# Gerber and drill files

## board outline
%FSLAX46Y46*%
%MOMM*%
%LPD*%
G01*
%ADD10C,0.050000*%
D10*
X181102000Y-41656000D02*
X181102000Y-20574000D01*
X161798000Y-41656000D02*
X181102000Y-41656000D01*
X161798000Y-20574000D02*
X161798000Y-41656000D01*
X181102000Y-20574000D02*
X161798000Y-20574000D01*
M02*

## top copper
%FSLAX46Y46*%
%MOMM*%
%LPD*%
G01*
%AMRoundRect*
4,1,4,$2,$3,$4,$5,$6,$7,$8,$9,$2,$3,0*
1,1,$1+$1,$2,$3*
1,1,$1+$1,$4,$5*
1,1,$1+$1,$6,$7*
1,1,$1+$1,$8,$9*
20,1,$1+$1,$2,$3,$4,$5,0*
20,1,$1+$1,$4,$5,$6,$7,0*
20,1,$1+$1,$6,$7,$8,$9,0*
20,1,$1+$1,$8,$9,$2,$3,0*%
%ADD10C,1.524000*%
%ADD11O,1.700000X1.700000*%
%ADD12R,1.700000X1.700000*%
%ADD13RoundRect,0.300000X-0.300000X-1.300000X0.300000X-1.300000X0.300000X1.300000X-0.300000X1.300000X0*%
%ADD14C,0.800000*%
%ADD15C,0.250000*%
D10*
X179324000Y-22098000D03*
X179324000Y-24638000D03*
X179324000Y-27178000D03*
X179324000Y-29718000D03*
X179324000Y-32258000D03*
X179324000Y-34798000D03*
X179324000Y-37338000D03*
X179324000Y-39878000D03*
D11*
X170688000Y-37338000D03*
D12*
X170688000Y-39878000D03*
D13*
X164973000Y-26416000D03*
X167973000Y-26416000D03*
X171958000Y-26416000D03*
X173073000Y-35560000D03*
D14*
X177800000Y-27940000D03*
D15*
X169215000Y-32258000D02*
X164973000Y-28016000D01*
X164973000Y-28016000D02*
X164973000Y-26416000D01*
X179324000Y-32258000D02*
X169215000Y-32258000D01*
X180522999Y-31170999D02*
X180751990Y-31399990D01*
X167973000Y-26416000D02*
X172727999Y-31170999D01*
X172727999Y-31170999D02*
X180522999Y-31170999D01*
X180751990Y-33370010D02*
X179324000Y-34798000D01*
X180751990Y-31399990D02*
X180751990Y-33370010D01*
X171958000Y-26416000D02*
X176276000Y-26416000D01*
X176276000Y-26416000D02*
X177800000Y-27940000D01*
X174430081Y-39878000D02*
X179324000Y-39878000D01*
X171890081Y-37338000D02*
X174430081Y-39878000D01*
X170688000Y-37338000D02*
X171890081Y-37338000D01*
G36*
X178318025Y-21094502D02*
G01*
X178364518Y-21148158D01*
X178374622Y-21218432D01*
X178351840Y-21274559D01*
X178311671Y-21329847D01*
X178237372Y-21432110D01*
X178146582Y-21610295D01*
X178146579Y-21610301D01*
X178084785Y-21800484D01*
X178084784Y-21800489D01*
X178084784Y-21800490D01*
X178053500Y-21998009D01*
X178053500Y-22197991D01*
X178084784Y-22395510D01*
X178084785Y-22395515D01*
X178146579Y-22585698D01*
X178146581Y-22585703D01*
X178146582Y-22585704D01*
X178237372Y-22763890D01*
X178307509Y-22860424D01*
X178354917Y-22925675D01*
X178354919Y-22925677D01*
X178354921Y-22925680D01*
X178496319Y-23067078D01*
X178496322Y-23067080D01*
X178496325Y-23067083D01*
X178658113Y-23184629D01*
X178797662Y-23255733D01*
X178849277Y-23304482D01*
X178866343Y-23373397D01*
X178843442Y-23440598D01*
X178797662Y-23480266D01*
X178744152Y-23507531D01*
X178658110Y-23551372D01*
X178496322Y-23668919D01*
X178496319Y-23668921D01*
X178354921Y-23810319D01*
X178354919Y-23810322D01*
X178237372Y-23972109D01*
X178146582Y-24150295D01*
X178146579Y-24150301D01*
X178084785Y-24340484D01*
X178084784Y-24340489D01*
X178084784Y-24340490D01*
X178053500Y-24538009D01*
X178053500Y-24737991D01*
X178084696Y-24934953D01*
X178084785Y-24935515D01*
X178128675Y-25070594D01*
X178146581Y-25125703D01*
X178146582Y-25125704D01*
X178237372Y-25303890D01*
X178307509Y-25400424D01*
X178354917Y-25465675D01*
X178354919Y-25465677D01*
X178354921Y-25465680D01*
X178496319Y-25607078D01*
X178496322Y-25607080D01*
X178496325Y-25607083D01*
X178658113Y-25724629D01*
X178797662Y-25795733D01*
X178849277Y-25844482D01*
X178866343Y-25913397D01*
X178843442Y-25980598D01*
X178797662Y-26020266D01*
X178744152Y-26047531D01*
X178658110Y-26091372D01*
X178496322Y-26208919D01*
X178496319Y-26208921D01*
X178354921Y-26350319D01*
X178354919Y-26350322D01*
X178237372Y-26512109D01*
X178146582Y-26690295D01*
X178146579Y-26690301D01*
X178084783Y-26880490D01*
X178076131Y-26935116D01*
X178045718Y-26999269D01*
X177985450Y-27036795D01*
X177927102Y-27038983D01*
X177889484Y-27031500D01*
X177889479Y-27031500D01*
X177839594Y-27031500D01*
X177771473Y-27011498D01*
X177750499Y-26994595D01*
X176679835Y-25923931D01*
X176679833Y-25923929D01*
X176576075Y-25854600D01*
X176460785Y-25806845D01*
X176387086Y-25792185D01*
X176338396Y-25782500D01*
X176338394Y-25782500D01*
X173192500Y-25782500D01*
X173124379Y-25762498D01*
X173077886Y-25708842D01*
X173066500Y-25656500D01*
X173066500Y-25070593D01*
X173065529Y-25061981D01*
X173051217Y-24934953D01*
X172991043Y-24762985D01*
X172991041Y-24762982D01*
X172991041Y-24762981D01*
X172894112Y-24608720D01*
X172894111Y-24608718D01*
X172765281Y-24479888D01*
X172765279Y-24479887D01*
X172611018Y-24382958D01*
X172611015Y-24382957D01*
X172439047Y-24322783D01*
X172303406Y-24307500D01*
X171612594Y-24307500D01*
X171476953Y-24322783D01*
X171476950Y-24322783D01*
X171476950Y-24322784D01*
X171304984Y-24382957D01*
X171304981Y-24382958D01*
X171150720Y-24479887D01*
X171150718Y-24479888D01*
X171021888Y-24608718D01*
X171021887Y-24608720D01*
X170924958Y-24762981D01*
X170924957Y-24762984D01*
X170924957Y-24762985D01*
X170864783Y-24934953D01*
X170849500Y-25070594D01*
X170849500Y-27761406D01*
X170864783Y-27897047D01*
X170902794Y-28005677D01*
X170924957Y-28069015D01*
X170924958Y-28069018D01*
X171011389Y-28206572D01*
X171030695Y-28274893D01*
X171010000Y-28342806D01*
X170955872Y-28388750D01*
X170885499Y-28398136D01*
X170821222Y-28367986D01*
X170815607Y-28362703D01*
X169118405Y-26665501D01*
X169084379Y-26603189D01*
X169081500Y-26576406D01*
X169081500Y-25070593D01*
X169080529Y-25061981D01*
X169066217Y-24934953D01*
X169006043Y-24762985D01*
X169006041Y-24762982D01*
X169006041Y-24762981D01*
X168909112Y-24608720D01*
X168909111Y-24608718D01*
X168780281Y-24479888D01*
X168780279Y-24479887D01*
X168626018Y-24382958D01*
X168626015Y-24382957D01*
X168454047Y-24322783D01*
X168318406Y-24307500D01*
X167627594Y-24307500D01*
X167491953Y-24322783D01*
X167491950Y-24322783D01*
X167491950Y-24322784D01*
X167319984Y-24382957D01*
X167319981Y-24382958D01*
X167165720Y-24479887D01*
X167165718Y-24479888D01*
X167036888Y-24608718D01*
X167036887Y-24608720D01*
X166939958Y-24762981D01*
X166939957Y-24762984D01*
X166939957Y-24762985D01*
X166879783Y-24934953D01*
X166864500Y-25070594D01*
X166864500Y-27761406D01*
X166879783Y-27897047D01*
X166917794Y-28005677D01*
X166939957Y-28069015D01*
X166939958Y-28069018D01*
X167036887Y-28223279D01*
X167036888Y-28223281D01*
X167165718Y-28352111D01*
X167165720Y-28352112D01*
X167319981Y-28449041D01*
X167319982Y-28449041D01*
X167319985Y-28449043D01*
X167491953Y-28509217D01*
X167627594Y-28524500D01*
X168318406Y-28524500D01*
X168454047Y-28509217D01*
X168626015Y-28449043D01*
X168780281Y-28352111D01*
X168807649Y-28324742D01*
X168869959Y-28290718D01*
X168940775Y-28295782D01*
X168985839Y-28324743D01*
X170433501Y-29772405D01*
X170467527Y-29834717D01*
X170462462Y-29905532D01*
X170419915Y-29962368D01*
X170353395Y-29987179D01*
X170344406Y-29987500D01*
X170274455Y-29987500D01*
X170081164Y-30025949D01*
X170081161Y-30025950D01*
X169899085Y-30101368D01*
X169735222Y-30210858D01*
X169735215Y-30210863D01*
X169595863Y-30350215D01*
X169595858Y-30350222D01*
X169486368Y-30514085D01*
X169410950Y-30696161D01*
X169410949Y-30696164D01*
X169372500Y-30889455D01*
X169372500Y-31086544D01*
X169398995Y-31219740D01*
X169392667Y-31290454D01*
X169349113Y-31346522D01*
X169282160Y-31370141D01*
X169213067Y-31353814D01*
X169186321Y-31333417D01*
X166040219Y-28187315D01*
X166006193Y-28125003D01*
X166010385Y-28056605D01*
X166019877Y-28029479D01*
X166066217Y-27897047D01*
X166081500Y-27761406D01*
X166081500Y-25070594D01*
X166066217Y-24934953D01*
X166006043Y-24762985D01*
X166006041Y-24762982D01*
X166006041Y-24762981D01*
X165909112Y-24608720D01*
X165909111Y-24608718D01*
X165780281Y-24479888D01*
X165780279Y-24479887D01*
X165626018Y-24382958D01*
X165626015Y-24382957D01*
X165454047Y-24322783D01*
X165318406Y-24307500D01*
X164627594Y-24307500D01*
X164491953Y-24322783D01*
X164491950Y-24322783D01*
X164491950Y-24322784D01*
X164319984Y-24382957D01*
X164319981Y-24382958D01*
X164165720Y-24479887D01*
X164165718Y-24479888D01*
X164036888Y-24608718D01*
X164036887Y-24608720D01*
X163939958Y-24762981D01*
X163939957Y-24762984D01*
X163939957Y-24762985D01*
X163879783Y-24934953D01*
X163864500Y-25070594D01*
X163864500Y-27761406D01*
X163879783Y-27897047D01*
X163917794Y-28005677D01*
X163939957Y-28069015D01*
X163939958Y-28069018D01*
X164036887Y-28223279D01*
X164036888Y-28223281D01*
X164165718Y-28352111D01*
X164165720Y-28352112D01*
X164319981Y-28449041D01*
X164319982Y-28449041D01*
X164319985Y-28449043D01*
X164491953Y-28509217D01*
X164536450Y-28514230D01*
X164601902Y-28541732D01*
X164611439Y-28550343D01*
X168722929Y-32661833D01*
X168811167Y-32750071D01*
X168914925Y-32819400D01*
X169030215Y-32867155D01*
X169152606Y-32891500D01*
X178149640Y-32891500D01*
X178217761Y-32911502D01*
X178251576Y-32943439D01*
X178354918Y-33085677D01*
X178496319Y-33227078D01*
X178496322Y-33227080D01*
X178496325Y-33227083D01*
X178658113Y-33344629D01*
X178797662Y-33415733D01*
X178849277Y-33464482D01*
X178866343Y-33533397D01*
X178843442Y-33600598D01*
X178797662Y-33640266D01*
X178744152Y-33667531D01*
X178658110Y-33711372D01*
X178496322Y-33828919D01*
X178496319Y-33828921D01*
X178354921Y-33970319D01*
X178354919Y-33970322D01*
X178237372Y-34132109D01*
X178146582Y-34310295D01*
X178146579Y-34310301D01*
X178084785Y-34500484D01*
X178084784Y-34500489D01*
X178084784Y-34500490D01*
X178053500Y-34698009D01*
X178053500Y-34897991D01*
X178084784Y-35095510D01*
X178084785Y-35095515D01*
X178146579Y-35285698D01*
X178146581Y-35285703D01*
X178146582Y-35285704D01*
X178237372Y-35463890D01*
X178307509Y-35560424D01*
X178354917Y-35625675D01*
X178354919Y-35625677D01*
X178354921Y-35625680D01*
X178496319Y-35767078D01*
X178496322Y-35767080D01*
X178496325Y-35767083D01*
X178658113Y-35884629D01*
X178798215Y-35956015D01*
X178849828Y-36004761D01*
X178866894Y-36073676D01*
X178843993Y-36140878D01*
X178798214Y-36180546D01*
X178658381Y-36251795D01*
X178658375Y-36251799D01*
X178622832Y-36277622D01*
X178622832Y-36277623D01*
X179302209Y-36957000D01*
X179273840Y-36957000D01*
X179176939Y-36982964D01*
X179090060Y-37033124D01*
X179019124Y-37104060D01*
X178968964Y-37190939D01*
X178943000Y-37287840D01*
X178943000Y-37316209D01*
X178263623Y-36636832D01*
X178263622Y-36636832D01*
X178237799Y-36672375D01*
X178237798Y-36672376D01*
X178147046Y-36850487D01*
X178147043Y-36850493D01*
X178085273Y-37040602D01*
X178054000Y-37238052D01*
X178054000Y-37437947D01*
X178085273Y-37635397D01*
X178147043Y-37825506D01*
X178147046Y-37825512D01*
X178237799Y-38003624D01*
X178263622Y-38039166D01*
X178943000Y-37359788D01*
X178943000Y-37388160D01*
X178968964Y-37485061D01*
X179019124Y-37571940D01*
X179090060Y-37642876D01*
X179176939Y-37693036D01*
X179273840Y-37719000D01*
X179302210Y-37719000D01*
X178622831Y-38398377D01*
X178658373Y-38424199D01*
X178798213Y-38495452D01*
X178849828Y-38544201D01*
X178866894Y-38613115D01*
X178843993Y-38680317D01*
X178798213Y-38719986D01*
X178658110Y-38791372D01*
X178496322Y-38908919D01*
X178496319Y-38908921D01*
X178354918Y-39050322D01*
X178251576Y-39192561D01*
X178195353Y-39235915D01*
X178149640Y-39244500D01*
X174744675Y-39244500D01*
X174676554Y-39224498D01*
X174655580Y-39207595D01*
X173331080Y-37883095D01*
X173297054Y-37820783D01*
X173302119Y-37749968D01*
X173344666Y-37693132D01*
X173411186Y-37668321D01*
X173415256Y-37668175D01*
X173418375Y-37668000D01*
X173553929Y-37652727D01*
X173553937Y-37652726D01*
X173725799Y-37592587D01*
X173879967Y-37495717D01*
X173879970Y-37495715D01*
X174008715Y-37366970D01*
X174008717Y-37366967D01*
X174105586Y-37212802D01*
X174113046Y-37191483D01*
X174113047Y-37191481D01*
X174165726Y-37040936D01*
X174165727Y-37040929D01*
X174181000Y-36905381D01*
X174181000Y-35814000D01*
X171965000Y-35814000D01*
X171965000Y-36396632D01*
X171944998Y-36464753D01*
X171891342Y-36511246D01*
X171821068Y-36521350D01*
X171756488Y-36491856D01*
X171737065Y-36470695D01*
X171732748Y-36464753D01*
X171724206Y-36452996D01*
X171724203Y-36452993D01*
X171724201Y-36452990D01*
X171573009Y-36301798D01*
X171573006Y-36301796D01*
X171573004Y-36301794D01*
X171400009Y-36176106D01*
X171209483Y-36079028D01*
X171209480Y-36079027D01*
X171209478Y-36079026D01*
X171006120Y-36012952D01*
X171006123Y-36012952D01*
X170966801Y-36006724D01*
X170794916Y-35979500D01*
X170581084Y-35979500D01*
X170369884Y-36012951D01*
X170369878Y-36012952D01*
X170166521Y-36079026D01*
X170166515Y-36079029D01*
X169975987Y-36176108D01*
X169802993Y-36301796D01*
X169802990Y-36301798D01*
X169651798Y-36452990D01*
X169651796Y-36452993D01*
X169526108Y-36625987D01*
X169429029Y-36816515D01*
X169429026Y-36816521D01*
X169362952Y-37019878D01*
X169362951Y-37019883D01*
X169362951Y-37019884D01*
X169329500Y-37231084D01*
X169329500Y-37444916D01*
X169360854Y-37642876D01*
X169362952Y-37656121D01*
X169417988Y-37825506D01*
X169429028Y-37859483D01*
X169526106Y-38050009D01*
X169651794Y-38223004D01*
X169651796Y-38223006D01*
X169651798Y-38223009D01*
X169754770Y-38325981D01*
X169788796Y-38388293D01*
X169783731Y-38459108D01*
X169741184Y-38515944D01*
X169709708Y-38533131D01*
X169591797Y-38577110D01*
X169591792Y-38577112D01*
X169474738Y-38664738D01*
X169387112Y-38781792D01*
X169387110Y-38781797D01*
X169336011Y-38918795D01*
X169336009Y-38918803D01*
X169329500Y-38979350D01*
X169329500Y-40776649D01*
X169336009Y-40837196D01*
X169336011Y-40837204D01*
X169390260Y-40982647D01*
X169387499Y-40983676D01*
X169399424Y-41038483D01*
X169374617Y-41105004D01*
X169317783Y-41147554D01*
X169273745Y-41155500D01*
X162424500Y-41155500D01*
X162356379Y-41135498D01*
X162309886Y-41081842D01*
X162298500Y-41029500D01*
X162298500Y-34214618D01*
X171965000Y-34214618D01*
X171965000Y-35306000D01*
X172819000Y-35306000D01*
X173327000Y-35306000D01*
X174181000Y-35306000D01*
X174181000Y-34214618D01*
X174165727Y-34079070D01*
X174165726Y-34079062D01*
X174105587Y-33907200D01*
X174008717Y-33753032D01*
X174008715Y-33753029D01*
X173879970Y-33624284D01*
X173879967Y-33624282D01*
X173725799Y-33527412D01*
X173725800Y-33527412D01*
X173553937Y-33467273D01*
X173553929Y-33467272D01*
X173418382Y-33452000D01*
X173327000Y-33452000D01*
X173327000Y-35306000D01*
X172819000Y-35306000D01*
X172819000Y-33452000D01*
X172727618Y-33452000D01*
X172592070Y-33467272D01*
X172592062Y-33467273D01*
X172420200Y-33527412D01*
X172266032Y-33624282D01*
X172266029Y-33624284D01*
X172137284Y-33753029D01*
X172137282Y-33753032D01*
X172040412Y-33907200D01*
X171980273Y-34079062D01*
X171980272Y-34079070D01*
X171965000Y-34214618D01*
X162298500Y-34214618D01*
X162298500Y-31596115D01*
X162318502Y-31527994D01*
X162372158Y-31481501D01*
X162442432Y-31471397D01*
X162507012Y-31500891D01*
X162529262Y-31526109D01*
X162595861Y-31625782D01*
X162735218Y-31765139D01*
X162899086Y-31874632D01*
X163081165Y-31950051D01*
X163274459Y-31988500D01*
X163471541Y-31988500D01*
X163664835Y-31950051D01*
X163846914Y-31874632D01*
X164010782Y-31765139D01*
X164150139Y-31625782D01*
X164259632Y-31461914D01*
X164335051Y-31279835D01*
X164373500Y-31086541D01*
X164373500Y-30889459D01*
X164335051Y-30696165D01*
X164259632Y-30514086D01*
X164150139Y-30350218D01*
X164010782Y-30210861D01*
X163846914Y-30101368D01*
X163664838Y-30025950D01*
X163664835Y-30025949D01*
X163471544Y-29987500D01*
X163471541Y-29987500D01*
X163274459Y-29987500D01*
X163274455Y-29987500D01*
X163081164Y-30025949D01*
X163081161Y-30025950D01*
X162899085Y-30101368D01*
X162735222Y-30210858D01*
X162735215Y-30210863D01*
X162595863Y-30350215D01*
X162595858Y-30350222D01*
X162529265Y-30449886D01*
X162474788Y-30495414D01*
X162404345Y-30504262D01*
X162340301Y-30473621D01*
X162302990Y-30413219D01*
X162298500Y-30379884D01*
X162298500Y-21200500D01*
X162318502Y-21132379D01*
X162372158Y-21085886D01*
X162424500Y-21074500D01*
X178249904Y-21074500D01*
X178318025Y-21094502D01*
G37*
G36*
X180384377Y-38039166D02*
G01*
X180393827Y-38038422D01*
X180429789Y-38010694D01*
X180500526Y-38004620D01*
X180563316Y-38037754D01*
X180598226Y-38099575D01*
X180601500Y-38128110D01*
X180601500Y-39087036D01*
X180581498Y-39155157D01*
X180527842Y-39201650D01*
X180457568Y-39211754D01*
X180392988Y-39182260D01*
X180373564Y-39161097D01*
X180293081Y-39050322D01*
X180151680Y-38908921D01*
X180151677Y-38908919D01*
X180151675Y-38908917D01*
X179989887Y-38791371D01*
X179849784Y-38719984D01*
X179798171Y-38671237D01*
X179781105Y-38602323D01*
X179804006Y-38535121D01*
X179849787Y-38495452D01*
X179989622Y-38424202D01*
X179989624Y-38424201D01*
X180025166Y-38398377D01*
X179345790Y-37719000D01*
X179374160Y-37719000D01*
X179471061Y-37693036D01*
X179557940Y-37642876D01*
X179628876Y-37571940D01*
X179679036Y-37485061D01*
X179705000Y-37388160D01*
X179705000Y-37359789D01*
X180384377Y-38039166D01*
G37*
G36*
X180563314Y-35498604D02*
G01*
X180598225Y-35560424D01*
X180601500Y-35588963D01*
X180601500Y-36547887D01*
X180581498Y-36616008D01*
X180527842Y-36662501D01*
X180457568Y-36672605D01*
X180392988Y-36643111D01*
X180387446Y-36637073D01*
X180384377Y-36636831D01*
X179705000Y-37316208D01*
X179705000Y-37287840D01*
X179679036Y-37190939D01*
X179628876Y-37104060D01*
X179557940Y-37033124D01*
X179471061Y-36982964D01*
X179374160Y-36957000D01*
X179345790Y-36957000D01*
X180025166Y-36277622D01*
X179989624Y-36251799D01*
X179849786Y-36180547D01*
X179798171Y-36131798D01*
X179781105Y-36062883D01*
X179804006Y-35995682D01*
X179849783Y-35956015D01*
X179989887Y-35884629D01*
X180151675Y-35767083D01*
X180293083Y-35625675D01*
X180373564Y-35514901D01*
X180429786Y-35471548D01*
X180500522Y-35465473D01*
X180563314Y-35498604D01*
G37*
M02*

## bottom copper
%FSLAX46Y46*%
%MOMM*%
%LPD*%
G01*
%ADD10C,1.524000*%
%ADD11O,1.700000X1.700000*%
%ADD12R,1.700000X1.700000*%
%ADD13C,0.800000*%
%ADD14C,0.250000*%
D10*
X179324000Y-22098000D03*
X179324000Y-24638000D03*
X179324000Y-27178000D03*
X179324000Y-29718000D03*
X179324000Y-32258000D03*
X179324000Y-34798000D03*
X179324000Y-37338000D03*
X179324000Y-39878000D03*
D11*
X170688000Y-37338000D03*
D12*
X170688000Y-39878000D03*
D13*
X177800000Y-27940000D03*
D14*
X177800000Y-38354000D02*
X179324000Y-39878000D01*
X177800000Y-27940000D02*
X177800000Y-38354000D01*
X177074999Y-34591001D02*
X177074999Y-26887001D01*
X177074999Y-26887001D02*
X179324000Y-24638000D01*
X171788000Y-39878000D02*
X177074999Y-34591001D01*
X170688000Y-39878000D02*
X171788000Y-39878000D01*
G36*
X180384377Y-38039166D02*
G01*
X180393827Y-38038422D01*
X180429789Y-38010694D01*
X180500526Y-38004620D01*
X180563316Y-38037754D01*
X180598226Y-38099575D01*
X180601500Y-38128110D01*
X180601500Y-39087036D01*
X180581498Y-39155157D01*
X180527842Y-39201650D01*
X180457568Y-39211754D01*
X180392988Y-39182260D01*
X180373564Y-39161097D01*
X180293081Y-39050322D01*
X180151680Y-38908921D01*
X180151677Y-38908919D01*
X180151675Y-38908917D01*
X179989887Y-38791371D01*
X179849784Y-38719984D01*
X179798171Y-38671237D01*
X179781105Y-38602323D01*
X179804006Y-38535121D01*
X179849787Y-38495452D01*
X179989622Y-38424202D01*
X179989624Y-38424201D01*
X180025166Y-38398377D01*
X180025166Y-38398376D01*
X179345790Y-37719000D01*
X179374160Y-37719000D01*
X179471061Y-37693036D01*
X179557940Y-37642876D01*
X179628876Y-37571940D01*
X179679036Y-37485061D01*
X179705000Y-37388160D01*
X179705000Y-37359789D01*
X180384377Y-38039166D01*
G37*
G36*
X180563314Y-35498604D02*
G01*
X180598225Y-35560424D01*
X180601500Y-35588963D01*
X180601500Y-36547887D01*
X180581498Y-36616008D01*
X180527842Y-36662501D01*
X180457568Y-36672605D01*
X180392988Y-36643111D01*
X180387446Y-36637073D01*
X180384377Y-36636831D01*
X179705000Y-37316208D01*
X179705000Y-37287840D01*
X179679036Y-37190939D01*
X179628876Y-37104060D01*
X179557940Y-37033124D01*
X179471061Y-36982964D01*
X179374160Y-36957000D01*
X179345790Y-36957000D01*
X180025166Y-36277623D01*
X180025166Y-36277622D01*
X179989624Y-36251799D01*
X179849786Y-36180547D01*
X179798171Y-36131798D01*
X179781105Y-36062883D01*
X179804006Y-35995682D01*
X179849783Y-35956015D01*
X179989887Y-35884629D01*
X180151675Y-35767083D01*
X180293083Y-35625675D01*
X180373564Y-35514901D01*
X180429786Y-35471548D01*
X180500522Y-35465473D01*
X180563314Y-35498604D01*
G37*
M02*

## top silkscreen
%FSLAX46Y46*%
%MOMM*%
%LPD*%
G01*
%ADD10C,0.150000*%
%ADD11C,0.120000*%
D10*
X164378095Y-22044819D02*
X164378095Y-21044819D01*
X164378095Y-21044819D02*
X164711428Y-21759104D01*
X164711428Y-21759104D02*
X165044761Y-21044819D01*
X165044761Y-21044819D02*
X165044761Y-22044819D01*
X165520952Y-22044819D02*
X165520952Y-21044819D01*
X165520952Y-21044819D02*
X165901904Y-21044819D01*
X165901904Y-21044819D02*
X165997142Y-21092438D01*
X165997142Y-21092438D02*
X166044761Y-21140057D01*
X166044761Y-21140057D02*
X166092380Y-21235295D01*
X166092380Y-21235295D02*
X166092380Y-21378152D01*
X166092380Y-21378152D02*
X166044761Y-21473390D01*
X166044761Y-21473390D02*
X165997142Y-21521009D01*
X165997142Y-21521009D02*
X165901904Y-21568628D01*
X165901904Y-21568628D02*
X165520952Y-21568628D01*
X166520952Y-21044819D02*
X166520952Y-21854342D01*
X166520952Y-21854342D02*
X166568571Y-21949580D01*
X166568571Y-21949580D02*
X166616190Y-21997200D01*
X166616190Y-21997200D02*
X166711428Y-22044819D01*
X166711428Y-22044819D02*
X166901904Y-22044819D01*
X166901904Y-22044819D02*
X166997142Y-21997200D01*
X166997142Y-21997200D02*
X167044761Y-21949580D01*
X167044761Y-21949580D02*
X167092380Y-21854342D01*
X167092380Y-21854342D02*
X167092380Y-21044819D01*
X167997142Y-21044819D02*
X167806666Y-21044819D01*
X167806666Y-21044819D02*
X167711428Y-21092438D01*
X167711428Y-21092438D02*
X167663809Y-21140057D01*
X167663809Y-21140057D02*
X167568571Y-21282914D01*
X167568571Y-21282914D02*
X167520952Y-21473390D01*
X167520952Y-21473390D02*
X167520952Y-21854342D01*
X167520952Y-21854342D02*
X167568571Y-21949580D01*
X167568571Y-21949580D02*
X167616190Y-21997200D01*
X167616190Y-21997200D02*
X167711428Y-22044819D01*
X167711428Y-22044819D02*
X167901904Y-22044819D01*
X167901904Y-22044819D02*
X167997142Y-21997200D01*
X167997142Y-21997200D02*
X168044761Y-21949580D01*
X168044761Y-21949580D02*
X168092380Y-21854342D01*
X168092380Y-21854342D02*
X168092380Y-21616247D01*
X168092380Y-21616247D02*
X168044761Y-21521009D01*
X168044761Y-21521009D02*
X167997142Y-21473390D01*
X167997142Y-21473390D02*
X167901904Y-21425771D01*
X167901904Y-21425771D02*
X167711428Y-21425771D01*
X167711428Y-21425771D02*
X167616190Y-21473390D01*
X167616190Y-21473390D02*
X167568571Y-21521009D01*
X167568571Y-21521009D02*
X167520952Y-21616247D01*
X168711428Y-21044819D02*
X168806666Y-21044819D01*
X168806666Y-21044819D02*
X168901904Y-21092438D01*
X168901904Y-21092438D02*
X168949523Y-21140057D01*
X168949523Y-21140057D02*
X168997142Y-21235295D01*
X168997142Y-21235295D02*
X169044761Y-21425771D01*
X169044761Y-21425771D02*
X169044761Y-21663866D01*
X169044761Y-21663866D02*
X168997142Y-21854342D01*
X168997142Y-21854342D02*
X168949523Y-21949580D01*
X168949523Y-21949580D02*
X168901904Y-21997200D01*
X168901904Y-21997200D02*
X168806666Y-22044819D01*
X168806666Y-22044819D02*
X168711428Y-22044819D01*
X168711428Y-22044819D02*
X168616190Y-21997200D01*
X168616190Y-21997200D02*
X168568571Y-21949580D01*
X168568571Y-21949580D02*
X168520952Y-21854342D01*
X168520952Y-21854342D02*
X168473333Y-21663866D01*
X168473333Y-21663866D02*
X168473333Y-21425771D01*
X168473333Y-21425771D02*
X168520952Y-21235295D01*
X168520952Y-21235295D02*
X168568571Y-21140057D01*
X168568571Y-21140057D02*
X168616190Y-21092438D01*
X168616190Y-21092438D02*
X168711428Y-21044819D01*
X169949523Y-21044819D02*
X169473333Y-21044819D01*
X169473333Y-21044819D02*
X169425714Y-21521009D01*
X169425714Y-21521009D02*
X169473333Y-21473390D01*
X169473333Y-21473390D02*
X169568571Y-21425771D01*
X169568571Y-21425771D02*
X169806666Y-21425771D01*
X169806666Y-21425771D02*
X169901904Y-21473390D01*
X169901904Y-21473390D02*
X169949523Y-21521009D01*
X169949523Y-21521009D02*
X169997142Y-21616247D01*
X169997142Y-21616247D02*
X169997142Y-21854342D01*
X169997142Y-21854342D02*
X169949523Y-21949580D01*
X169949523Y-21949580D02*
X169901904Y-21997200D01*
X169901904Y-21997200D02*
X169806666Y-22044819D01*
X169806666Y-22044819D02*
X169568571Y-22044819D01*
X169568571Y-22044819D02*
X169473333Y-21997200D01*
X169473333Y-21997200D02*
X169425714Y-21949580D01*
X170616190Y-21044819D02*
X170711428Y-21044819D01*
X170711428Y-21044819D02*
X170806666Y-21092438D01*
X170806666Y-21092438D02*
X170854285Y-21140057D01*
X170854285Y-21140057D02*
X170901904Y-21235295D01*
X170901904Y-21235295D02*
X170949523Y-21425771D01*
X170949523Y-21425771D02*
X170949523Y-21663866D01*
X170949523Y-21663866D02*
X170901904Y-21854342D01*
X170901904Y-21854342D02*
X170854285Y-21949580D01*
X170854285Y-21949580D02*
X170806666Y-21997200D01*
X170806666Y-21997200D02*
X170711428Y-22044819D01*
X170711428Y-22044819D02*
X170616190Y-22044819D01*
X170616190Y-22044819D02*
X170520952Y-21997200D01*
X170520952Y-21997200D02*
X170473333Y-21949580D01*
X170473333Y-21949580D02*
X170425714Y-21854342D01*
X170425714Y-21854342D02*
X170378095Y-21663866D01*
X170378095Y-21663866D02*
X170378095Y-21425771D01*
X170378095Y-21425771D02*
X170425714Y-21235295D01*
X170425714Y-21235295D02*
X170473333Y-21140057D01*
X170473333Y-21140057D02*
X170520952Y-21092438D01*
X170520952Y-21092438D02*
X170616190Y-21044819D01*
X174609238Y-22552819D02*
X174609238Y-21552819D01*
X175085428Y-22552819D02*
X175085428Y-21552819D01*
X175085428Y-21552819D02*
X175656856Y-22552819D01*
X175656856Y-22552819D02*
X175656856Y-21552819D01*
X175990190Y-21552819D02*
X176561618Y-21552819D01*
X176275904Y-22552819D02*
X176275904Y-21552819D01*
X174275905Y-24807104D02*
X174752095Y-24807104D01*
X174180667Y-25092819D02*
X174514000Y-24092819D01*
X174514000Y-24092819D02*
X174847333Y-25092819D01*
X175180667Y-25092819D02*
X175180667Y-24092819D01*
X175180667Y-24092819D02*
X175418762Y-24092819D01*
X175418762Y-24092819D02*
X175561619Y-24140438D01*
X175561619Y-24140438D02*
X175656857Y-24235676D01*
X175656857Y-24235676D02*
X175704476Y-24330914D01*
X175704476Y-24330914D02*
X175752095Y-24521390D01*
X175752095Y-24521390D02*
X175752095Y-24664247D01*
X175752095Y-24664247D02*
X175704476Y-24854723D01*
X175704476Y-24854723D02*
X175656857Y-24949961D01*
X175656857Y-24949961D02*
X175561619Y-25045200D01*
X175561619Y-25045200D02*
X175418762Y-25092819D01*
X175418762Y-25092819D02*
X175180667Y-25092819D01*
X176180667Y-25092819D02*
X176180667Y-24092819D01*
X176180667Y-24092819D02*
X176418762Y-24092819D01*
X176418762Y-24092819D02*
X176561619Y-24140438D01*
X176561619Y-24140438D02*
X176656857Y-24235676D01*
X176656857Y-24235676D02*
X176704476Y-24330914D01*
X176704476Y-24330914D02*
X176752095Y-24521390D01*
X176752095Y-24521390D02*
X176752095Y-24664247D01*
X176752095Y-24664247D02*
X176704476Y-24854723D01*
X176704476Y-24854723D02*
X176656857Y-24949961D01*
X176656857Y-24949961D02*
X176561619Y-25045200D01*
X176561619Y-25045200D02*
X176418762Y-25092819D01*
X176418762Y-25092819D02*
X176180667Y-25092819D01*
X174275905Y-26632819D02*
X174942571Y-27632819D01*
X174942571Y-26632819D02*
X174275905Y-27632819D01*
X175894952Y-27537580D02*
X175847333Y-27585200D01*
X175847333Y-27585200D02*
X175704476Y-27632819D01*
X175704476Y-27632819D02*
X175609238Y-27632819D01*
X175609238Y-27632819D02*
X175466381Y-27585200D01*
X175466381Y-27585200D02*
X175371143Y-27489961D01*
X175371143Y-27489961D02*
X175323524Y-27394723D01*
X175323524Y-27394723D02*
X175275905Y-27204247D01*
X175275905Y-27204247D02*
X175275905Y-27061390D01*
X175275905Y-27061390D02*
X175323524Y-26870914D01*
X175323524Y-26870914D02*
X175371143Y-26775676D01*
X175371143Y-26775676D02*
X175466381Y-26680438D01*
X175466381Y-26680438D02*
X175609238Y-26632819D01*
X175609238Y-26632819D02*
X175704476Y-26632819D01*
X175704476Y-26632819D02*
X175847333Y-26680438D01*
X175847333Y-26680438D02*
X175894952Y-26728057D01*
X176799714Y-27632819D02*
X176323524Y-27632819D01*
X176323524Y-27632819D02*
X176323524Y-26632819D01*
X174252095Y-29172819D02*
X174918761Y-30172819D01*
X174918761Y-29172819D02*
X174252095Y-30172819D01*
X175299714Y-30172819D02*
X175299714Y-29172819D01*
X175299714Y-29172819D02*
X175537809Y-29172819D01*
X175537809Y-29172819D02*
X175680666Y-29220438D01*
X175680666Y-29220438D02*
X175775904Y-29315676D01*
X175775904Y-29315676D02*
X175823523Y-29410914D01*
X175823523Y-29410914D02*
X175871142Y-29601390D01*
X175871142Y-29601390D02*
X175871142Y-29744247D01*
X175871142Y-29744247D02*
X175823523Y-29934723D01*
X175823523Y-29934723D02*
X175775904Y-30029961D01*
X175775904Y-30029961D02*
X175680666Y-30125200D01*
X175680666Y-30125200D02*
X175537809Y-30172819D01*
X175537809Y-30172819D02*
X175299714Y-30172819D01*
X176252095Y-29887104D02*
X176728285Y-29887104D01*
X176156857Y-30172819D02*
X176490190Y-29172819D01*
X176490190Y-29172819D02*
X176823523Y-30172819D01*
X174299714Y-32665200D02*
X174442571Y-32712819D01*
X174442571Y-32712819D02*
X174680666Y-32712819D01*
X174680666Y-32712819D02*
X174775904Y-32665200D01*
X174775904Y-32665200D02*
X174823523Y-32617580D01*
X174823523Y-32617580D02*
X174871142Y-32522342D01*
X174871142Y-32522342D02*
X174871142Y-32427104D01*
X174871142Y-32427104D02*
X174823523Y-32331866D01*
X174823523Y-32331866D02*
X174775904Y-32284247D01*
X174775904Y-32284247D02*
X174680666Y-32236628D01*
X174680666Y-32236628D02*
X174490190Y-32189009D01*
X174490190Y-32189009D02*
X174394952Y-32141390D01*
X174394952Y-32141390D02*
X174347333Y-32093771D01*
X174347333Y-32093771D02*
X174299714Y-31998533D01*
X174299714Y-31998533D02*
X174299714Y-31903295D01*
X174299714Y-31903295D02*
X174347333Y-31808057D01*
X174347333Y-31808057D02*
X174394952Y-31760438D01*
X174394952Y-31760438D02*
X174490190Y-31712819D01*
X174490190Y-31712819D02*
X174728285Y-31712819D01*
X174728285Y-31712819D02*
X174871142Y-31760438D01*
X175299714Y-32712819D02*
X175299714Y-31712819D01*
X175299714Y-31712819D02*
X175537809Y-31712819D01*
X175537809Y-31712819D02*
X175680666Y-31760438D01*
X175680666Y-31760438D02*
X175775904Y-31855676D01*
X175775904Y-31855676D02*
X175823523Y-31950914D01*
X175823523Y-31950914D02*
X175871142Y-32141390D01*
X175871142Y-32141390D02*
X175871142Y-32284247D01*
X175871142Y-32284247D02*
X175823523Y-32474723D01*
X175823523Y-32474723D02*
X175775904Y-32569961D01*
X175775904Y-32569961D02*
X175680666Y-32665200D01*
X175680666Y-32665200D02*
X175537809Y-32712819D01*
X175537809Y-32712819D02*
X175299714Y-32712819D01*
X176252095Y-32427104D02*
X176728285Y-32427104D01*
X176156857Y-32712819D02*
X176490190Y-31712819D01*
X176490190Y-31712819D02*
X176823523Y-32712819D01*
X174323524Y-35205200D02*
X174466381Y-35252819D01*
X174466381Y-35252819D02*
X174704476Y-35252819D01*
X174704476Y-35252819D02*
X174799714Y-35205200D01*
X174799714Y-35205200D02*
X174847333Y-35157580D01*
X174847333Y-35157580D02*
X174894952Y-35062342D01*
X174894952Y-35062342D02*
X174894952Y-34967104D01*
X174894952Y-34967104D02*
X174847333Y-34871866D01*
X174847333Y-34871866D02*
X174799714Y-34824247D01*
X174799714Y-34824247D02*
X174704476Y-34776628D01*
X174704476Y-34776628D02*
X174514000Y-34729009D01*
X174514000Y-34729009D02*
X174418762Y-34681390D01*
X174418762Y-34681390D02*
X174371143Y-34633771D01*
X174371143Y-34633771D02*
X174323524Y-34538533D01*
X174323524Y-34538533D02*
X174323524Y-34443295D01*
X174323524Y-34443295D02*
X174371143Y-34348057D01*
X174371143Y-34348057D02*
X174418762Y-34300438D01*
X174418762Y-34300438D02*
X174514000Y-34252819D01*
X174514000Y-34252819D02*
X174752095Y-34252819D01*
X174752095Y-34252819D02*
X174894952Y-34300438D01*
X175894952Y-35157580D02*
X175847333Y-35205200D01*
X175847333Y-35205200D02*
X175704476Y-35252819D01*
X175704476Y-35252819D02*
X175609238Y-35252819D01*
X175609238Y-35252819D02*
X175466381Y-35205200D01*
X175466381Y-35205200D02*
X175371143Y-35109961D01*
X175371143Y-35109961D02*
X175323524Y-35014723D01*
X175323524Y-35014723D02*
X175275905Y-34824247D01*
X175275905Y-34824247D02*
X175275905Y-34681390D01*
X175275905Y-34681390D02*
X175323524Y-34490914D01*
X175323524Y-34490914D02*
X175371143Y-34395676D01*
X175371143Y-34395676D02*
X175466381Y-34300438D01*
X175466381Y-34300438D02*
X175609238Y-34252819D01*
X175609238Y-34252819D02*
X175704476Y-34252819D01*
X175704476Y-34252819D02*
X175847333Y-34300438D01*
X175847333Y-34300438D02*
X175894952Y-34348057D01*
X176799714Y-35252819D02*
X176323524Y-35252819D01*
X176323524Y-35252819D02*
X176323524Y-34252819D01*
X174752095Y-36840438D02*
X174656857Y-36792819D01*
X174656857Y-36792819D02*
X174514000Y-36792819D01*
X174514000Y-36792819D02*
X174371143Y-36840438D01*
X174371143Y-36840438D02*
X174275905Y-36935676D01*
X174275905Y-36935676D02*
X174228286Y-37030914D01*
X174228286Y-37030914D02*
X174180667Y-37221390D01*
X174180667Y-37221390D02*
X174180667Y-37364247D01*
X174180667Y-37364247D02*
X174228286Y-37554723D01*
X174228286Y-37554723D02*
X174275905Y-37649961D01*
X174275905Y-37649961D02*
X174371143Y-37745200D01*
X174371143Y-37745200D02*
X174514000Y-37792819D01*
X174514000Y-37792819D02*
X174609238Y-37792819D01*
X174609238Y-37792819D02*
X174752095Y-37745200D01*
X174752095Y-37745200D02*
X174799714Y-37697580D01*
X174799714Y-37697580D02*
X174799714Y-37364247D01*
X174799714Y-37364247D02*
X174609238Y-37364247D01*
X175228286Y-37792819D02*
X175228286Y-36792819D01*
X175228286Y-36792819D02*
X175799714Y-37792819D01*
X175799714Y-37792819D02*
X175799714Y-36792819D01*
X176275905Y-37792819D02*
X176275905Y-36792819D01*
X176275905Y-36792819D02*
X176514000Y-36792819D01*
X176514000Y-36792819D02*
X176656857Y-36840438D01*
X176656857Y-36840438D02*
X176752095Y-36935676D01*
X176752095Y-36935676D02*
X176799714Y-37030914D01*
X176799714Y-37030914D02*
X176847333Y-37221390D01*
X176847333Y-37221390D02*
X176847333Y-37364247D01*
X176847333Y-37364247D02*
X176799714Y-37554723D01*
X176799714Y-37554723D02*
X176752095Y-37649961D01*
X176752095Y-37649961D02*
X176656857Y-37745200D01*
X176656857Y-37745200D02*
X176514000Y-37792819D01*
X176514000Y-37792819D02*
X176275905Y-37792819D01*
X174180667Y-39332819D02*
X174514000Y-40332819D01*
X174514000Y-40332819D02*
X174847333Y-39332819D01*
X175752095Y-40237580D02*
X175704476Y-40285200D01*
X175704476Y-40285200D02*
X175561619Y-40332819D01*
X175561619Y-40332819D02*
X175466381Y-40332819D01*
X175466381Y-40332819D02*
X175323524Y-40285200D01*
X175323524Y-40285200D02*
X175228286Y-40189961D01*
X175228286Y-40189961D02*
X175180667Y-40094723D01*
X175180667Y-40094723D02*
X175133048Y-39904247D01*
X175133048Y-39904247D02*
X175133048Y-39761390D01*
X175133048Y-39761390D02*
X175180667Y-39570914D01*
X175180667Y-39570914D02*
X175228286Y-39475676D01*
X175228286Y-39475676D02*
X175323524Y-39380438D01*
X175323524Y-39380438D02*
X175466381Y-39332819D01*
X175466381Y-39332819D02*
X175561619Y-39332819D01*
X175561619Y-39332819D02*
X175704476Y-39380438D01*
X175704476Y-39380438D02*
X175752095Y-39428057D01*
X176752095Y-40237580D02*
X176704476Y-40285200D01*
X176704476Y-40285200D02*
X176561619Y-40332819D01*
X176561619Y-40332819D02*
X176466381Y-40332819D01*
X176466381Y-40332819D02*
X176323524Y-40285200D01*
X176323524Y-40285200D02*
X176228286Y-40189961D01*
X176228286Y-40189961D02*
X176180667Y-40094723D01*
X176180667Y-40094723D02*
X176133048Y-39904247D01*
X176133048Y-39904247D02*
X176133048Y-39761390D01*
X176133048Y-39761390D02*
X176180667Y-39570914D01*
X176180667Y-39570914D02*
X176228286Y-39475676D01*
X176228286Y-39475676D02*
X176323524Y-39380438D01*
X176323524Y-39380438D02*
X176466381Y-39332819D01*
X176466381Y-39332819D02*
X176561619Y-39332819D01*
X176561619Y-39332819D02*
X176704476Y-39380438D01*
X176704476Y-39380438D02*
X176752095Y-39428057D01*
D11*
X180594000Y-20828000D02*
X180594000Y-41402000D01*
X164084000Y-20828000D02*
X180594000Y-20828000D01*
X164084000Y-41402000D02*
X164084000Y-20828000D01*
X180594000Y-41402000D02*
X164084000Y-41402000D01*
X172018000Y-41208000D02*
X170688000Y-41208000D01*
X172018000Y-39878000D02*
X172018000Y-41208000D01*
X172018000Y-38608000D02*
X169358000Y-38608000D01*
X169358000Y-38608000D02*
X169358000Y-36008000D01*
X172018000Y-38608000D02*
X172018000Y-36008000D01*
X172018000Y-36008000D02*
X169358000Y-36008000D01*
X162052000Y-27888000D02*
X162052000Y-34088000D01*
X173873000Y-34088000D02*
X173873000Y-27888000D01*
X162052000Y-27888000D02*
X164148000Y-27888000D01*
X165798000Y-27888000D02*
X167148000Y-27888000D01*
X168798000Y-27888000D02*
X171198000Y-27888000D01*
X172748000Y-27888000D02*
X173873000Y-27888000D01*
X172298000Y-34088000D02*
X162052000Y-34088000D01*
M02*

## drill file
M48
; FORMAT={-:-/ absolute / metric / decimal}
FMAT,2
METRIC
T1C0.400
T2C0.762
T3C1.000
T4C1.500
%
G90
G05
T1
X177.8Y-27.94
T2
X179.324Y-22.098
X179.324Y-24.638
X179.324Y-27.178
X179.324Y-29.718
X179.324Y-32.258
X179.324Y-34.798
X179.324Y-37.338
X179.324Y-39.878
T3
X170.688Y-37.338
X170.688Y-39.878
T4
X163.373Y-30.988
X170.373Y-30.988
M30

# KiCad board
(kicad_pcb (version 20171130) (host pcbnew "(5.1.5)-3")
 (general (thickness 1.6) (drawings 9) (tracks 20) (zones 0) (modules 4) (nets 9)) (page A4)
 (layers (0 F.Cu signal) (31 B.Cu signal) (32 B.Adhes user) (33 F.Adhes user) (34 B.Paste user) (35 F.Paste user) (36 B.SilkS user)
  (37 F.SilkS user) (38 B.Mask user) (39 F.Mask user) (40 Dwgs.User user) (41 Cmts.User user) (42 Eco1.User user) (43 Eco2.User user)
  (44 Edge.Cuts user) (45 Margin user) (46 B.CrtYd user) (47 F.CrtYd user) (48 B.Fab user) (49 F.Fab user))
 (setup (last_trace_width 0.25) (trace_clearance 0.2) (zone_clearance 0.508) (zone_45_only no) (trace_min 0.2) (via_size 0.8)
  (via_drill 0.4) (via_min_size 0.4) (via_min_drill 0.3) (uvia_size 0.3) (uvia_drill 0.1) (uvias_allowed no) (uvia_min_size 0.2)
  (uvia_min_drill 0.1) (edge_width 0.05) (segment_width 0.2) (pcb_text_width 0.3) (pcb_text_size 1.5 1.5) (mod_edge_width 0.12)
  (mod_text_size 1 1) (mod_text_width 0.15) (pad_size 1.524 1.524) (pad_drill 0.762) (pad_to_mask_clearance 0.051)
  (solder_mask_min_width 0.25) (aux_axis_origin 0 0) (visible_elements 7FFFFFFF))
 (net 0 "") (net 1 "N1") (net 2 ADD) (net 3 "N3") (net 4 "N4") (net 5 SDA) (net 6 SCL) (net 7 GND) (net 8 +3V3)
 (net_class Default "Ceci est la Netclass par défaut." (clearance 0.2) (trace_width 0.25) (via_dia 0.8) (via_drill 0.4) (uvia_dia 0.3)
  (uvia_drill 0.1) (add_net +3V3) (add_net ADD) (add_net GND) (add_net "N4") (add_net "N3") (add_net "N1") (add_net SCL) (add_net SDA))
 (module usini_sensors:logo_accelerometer (layer B.Cu) (at 165.608 24.384 180)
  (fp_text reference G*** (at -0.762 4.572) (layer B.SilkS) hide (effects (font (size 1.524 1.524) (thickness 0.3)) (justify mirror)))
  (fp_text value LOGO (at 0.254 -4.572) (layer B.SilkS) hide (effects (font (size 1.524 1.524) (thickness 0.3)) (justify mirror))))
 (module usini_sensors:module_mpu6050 (layer F.Cu) (at 179.324 22.098 180)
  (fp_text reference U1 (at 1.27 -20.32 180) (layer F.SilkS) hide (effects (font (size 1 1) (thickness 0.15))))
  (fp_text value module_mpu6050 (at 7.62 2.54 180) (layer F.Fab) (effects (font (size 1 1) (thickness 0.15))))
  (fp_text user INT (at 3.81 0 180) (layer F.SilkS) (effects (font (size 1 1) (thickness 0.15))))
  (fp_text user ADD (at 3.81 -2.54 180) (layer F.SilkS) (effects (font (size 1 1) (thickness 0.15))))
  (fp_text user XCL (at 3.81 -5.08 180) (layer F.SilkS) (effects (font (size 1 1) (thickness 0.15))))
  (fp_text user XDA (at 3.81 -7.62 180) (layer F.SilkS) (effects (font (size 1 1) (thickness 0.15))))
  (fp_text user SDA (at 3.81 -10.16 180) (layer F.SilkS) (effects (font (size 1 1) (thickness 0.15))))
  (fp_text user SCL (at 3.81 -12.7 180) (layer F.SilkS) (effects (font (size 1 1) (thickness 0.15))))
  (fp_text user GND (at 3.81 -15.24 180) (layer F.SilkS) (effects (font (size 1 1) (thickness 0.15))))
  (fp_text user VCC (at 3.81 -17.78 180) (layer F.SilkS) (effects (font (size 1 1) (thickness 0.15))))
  (fp_line (start -1.27 1.27) (end -1.27 -19.304) (layer F.SilkS) (width 0.12))
  (fp_line (start 15.24 1.27) (end -1.27 1.27) (layer F.SilkS) (width 0.12))
  (fp_line (start 15.24 -19.304) (end 15.24 1.27) (layer F.SilkS) (width 0.12))
  (fp_line (start -1.27 -19.304) (end 15.24 -19.304) (layer F.SilkS) (width 0.12))
  (pad 8 thru_hole circle (at 0 0 180) (size 1.524 1.524) (drill 0.762) (layers *.Cu *.Mask) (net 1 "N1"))
  (pad 7 thru_hole circle (at 0 -2.54 180) (size 1.524 1.524) (drill 0.762) (layers *.Cu *.Mask) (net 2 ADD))
  (pad 6 thru_hole circle (at 0 -5.08 180) (size 1.524 1.524) (drill 0.762) (layers *.Cu *.Mask) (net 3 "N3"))
  (pad 5 thru_hole circle (at 0 -7.62 180) (size 1.524 1.524) (drill 0.762) (layers *.Cu *.Mask) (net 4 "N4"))
  (pad 4 thru_hole circle (at 0 -10.16 180) (size 1.524 1.524) (drill 0.762) (layers *.Cu *.Mask) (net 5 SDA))
  (pad 3 thru_hole circle (at 0 -12.7 180) (size 1.524 1.524) (drill 0.762) (layers *.Cu *.Mask) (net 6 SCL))
  (pad 2 thru_hole circle (at 0 -15.24 180) (size 1.524 1.524) (drill 0.762) (layers *.Cu *.Mask) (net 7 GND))
  (pad 1 thru_hole circle (at 0 -17.78 180) (size 1.524 1.524) (drill 0.762) (layers *.Cu *.Mask) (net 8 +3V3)))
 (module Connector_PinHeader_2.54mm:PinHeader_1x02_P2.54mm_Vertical (layer F.Cu) (at 170.688 39.878 180)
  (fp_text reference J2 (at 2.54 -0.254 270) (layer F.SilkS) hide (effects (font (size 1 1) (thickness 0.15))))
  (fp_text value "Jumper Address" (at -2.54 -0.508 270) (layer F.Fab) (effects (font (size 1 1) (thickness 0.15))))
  (fp_line (start -1.33 -1.33) (end 0 -1.33) (layer F.SilkS) (width 0.12))
  (fp_line (start -1.33 0) (end -1.33 -1.33) (layer F.SilkS) (width 0.12))
  (fp_line (start -1.33 1.27) (end 1.33 1.27) (layer F.SilkS) (width 0.12))
  (fp_line (start 1.33 1.27) (end 1.33 3.87) (layer F.SilkS) (width 0.12))
  (fp_line (start -1.33 1.27) (end -1.33 3.87) (layer F.SilkS) (width 0.12))
  (fp_line (start -1.33 3.87) (end 1.33 3.87) (layer F.SilkS) (width 0.12))
  (pad 2 thru_hole oval (at 0 2.54 180) (size 1.7 1.7) (drill 1) (layers *.Cu *.Mask) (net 8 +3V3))
  (pad 1 thru_hole rect (at 0 0 180) (size 1.7 1.7) (drill 1) (layers *.Cu *.Mask) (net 2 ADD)))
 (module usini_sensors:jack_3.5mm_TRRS (layer F.Cu) (at 168.148 30.988)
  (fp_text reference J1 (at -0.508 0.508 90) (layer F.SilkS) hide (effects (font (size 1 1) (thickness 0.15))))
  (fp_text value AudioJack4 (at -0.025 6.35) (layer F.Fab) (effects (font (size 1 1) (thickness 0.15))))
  (fp_line (start -6.096 -3.1) (end -6.096 3.1) (layer F.SilkS) (width 0.12))
  (fp_line (start 5.725 3.1) (end 5.725 -3.1) (layer F.SilkS) (width 0.12))
  (fp_line (start -6.096 -3.1) (end -4 -3.1) (layer F.SilkS) (width 0.12))
  (fp_line (start -2.35 -3.1) (end -1 -3.1) (layer F.SilkS) (width 0.12))
  (fp_line (start 0.65 -3.1) (end 3.05 -3.1) (layer F.SilkS) (width 0.12))
  (fp_line (start 4.6 -3.1) (end 5.725 -3.1) (layer F.SilkS) (width 0.12))
  (fp_line (start 4.15 3.1) (end -6.096 3.1) (layer F.SilkS) (width 0.12))
  (pad "" np_thru_hole circle (at 2.225 0) (size 1.5 1.5) (drill 1.5) (layers *.Cu *.Mask))
  (pad "" np_thru_hole circle (at -4.775 0) (size 1.5 1.5) (drill 1.5) (layers *.Cu *.Mask))
  (pad R2 smd roundrect (at -3.175 -4.572) (size 1.2 3.2) (layers F.Cu F.Paste F.Mask) (roundrect_rratio 0.25) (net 5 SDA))
  (pad R1 smd roundrect (at -0.175 -4.572) (size 1.2 3.2) (layers F.Cu F.Paste F.Mask) (roundrect_rratio 0.25) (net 6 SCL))
  (pad T smd roundrect (at 3.81 -4.572) (size 1.2 3.2) (layers F.Cu F.Paste F.Mask) (roundrect_rratio 0.25) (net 8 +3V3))
  (pad S smd roundrect (at 4.925 4.572) (size 1.2 3.2) (layers F.Cu F.Paste F.Mask) (roundrect_rratio 0.25) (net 7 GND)))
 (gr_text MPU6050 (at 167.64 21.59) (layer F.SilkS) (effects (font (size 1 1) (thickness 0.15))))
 (gr_line (start 181.102 41.656) (end 181.102 20.574) (layer Edge.Cuts) (width 0.05))
 (gr_line (start 161.798 41.656) (end 181.102 41.656) (layer Edge.Cuts) (width 0.05))
 (gr_line (start 161.798 20.574) (end 161.798 41.656) (layer Edge.Cuts) (width 0.05))
 (gr_line (start 181.102 20.574) (end 161.798 20.574) (layer Edge.Cuts) (width 0.05))
 (segment (start 169.215 32.258) (end 164.973 28.016) (width 0.25) (layer F.Cu) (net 5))
 (segment (start 164.973 28.016) (end 164.973 26.416) (width 0.25) (layer F.Cu) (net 5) (status 20))
 (segment (start 179.324 32.258) (end 169.215 32.258) (width 0.25) (layer F.Cu) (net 5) (status 10))
 (segment (start 180.522999 31.170999) (end 180.75199 31.39999) (width 0.25) (layer F.Cu) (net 6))
 (segment (start 167.973 26.416) (end 172.727999 31.170999) (width 0.25) (layer F.Cu) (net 6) (status 10))
 (segment (start 172.727999 31.170999) (end 180.522999 31.170999) (width 0.25) (layer F.Cu) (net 6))
 (segment (start 180.75199 33.37001) (end 179.324 34.798) (width 0.25) (layer F.Cu) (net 6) (status 20))
 (segment (start 180.75199 31.39999) (end 180.75199 33.37001) (width 0.25) (layer F.Cu) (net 6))
 (via (at 177.8 27.94) (size 0.8) (drill 0.4) (layers F.Cu B.Cu) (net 8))
 (segment (start 171.958 26.416) (end 176.276 26.416) (width 0.25) (layer F.Cu) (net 8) (status 10))
 (segment (start 176.276 26.416) (end 177.8 27.94) (width 0.25) (layer F.Cu) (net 8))
 (segment (start 177.8 38.354) (end 179.324 39.878) (width 0.25) (layer B.Cu) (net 8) (status 20))
 (segment (start 177.8 27.94) (end 177.8 38.354) (width 0.25) (layer B.Cu) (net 8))
 (segment (start 174.430081 39.878) (end 179.324 39.878) (width 0.25) (layer F.Cu) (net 8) (status 20))
 (segment (start 171.890081 37.338) (end 174.430081 39.878) (width 0.25) (layer F.Cu) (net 8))
 (segment (start 170.688 37.338) (end 171.890081 37.338) (width 0.25) (layer F.Cu) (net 8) (status 10))
 (segment (start 177.074999 34.591001) (end 177.074999 26.887001) (width 0.25) (layer B.Cu) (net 2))
 (segment (start 177.074999 26.887001) (end 179.324 24.638) (width 0.25) (layer B.Cu) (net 2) (status 20))
 (segment (start 171.788 39.878) (end 177.074999 34.591001) (width 0.25) (layer B.Cu) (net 2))
 (segment (start 170.688 39.878) (end 171.788 39.878) (width 0.25) (layer B.Cu) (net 2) (status 10))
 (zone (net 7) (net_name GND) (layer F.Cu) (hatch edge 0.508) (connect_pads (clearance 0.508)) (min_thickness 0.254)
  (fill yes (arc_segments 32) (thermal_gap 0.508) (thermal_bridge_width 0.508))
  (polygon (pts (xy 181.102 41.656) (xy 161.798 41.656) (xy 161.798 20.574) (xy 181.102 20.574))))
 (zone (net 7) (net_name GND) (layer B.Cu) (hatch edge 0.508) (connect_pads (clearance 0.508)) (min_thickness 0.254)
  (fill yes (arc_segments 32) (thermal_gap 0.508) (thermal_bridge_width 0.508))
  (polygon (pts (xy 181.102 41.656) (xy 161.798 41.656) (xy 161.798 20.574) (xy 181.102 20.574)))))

